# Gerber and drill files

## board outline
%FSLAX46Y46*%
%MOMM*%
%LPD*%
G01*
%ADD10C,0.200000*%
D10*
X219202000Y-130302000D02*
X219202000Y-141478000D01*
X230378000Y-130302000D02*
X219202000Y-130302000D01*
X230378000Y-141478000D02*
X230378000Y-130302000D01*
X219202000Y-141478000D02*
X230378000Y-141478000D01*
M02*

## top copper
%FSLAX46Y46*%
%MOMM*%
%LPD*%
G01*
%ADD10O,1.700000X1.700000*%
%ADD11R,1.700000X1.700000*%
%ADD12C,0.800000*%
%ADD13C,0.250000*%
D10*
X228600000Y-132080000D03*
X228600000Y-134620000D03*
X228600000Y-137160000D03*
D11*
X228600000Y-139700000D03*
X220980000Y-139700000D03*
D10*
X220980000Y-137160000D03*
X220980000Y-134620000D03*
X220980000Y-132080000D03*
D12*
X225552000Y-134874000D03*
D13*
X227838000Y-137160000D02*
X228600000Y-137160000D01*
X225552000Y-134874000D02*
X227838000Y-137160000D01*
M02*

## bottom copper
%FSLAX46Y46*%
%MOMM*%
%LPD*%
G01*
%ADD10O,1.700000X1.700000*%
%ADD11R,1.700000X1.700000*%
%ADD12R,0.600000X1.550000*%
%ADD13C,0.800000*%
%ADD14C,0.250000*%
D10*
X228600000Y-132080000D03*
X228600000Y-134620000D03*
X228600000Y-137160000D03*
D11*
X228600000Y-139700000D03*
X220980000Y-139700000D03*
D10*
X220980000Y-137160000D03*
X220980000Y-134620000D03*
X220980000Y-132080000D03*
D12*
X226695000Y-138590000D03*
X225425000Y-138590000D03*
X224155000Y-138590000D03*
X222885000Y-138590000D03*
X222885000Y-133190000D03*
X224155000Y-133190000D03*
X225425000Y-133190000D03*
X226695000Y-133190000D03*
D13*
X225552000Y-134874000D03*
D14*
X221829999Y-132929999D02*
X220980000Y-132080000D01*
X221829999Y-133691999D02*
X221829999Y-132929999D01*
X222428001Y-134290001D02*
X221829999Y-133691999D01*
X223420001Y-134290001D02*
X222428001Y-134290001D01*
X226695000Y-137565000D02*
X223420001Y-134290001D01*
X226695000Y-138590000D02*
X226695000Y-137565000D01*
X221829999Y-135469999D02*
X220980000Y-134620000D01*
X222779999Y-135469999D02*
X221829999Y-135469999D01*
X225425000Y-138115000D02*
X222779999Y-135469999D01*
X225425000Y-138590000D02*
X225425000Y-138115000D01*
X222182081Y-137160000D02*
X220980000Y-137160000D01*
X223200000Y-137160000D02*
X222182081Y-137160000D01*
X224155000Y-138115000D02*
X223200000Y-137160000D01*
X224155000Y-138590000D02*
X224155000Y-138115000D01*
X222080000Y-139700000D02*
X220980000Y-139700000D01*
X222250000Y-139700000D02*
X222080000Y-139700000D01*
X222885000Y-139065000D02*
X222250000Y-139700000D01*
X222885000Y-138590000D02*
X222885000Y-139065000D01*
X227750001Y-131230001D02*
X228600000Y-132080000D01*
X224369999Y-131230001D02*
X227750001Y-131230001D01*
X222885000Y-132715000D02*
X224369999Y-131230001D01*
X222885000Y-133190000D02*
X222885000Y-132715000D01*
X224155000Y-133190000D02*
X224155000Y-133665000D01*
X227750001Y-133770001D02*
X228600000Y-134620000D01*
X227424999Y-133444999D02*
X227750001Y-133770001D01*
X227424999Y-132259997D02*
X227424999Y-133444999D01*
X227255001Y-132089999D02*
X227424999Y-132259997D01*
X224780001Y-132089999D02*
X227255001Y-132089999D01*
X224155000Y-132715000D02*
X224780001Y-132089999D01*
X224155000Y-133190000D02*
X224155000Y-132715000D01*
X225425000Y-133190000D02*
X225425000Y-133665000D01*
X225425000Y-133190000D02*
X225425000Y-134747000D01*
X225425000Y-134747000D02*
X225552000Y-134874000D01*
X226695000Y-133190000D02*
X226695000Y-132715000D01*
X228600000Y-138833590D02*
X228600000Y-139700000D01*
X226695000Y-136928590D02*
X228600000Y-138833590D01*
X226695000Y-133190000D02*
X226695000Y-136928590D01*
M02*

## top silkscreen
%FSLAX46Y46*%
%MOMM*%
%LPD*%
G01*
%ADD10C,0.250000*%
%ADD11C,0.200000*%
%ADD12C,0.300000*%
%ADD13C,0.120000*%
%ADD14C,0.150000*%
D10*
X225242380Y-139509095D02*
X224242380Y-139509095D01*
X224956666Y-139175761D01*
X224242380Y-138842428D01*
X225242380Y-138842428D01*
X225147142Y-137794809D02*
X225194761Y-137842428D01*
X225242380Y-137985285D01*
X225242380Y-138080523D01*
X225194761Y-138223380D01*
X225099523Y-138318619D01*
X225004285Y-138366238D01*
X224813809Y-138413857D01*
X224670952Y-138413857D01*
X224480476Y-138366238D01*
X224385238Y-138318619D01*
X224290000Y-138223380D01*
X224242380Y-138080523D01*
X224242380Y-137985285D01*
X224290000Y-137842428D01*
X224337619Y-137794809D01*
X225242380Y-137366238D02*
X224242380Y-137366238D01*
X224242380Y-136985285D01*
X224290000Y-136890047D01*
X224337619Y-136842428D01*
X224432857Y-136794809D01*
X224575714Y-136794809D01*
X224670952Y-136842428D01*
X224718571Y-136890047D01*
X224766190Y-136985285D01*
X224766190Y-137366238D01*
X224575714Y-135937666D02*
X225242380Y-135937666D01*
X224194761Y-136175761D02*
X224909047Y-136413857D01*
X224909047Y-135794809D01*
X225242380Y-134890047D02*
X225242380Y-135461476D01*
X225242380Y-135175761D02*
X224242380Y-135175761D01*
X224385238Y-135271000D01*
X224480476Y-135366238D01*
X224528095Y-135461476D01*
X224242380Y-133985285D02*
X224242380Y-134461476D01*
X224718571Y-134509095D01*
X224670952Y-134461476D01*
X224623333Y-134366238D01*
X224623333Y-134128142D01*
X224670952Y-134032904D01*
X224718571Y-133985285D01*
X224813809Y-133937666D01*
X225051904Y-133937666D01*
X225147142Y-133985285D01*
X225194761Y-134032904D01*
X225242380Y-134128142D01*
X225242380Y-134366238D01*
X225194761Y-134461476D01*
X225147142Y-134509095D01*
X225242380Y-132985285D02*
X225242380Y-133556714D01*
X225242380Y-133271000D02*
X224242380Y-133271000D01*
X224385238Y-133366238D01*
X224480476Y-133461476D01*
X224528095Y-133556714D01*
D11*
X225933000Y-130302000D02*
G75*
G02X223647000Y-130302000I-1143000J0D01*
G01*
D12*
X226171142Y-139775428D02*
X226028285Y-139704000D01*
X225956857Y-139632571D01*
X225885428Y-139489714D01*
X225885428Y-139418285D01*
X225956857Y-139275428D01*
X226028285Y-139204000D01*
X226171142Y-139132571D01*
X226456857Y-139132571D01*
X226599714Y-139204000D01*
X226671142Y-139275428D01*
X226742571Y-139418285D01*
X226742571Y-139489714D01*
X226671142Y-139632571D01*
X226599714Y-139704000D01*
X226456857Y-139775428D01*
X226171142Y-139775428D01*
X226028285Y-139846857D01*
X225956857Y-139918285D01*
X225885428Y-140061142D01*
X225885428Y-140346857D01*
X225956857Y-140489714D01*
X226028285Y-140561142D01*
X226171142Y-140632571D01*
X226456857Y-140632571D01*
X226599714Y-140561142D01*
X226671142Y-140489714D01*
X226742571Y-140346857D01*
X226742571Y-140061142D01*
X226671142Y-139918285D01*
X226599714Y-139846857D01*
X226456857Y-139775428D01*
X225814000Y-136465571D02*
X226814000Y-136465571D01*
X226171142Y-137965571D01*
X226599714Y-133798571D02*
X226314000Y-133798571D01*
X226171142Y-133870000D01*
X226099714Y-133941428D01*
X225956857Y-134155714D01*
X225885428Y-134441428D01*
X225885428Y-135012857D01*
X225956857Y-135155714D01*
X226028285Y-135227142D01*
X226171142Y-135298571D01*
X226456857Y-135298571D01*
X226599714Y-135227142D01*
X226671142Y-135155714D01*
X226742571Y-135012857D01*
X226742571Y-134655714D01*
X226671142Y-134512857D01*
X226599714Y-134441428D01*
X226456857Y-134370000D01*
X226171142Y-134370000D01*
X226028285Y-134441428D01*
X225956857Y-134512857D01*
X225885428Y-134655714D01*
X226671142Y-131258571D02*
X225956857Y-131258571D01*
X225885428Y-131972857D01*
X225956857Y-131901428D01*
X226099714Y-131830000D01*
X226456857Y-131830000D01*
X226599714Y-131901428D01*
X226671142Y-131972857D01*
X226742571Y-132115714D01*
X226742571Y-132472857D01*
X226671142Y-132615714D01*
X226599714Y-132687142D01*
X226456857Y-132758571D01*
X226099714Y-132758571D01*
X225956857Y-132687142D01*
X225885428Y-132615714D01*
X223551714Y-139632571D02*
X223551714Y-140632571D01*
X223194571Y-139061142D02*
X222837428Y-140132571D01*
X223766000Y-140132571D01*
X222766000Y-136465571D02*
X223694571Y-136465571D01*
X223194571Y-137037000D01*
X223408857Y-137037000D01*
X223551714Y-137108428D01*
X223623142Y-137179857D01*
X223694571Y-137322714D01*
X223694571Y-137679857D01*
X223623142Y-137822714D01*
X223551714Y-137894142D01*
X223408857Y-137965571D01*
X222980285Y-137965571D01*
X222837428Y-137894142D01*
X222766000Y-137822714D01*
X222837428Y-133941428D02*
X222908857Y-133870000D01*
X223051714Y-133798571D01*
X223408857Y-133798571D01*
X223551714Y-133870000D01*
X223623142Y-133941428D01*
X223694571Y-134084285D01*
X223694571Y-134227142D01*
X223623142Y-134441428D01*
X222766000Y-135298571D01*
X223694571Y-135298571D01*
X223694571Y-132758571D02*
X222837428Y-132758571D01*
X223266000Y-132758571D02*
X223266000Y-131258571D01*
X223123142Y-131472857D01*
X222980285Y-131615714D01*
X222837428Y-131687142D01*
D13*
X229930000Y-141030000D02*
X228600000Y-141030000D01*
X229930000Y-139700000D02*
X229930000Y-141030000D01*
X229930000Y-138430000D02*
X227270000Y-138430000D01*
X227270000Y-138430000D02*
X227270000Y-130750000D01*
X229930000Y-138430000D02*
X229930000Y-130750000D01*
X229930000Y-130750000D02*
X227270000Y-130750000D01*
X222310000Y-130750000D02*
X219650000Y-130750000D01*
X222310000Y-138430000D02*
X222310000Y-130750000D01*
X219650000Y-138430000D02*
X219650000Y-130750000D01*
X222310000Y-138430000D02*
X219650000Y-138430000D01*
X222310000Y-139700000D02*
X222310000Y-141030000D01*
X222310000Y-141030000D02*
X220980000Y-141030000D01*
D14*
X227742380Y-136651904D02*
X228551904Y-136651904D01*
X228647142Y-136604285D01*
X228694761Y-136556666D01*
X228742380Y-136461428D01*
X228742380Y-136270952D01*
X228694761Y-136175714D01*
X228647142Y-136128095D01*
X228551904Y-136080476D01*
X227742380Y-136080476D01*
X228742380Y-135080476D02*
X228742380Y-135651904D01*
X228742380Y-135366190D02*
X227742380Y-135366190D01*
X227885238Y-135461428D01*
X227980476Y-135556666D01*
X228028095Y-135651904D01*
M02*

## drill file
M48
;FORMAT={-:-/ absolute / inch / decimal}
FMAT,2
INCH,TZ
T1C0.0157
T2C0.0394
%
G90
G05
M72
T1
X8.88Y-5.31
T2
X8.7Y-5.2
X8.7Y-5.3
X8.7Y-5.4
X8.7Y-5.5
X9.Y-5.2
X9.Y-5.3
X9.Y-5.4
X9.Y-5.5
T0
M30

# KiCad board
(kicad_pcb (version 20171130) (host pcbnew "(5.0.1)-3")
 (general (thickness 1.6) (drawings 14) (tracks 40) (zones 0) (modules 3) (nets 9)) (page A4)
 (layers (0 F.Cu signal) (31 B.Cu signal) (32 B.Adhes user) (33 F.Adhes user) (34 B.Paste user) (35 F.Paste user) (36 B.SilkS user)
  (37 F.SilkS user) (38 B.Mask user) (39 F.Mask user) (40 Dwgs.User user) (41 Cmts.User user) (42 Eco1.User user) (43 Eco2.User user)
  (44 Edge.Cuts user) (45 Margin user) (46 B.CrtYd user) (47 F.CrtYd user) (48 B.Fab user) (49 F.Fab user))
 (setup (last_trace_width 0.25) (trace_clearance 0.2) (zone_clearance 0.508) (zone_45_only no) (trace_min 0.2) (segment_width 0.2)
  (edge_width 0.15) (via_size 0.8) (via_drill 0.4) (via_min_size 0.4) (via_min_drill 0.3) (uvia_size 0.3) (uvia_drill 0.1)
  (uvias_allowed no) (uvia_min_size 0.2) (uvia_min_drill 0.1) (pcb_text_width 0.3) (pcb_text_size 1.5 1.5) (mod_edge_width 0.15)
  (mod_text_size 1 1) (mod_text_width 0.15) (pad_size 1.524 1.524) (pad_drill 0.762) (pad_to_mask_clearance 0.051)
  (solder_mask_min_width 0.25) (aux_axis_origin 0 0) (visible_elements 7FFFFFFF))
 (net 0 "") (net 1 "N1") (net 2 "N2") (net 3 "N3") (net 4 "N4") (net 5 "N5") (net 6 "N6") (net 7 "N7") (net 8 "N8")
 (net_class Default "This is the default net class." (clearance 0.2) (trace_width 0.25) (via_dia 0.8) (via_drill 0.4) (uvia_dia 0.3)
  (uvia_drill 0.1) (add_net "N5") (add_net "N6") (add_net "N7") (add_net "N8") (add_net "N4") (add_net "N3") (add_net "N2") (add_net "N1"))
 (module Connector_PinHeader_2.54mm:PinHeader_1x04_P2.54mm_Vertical (layer F.Cu) (at 228.6 139.7 180)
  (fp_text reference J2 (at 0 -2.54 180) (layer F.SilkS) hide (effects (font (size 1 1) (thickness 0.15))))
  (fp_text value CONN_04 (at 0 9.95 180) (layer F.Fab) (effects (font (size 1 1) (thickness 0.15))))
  (fp_line (start -1.33 -1.33) (end 0 -1.33) (layer F.SilkS) (width 0.12))
  (fp_line (start -1.33 0) (end -1.33 -1.33) (layer F.SilkS) (width 0.12))
  (fp_line (start -1.33 1.27) (end 1.33 1.27) (layer F.SilkS) (width 0.12))
  (fp_line (start 1.33 1.27) (end 1.33 8.95) (layer F.SilkS) (width 0.12))
  (fp_line (start -1.33 1.27) (end -1.33 8.95) (layer F.SilkS) (width 0.12))
  (fp_line (start -1.33 8.95) (end 1.33 8.95) (layer F.SilkS) (width 0.12))
  (pad 4 thru_hole oval (at 0 7.62 180) (size 1.7 1.7) (drill 1) (layers *.Cu *.Mask) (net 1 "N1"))
  (pad 3 thru_hole oval (at 0 5.08 180) (size 1.7 1.7) (drill 1) (layers *.Cu *.Mask) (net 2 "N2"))
  (pad 2 thru_hole oval (at 0 2.54 180) (size 1.7 1.7) (drill 1) (layers *.Cu *.Mask) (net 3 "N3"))
  (pad 1 thru_hole rect (at 0 0 180) (size 1.7 1.7) (drill 1) (layers *.Cu *.Mask) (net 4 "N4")))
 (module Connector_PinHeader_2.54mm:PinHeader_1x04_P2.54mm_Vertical (layer F.Cu) (at 220.98 139.7 180)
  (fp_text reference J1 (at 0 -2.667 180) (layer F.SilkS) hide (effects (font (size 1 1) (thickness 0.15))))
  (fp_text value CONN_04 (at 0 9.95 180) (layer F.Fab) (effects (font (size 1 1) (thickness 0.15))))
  (fp_line (start -1.33 8.95) (end 1.33 8.95) (layer F.SilkS) (width 0.12))
  (fp_line (start -1.33 1.27) (end -1.33 8.95) (layer F.SilkS) (width 0.12))
  (fp_line (start 1.33 1.27) (end 1.33 8.95) (layer F.SilkS) (width 0.12))
  (fp_line (start -1.33 1.27) (end 1.33 1.27) (layer F.SilkS) (width 0.12))
  (fp_line (start -1.33 0) (end -1.33 -1.33) (layer F.SilkS) (width 0.12))
  (fp_line (start -1.33 -1.33) (end 0 -1.33) (layer F.SilkS) (width 0.12))
  (pad 1 thru_hole rect (at 0 0 180) (size 1.7 1.7) (drill 1) (layers *.Cu *.Mask) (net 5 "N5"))
  (pad 2 thru_hole oval (at 0 2.54 180) (size 1.7 1.7) (drill 1) (layers *.Cu *.Mask) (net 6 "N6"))
  (pad 3 thru_hole oval (at 0 5.08 180) (size 1.7 1.7) (drill 1) (layers *.Cu *.Mask) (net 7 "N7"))
  (pad 4 thru_hole oval (at 0 7.62 180) (size 1.7 1.7) (drill 1) (layers *.Cu *.Mask) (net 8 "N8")))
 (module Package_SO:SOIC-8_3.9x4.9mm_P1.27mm (layer B.Cu) (at 224.79 135.89 90)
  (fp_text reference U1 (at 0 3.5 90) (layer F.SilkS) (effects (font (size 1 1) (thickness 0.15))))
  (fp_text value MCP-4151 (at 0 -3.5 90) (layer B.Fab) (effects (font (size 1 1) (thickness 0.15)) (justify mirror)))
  (pad 1 smd rect (at -2.7 1.905 90) (size 1.55 0.6) (layers B.Cu B.Paste B.Mask) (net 8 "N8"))
  (pad 2 smd rect (at -2.7 0.635 90) (size 1.55 0.6) (layers B.Cu B.Paste B.Mask) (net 7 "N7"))
  (pad 3 smd rect (at -2.7 -0.635 90) (size 1.55 0.6) (layers B.Cu B.Paste B.Mask) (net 6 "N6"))
  (pad 4 smd rect (at -2.7 -1.905 90) (size 1.55 0.6) (layers B.Cu B.Paste B.Mask) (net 5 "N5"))
  (pad 5 smd rect (at 2.7 -1.905 90) (size 1.55 0.6) (layers B.Cu B.Paste B.Mask) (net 1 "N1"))
  (pad 6 smd rect (at 2.7 -0.635 90) (size 1.55 0.6) (layers B.Cu B.Paste B.Mask) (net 2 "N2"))
  (pad 7 smd rect (at 2.7 0.635 90) (size 1.55 0.6) (layers B.Cu B.Paste B.Mask) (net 3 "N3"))
  (pad 8 smd rect (at 2.7 1.905 90) (size 1.55 0.6) (layers B.Cu B.Paste B.Mask) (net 4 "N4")))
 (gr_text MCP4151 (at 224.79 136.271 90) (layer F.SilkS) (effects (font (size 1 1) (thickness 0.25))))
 (gr_arc (start 224.79 130.302) (end 223.647 130.302) (angle -180) (layer F.SilkS) (width 0.2))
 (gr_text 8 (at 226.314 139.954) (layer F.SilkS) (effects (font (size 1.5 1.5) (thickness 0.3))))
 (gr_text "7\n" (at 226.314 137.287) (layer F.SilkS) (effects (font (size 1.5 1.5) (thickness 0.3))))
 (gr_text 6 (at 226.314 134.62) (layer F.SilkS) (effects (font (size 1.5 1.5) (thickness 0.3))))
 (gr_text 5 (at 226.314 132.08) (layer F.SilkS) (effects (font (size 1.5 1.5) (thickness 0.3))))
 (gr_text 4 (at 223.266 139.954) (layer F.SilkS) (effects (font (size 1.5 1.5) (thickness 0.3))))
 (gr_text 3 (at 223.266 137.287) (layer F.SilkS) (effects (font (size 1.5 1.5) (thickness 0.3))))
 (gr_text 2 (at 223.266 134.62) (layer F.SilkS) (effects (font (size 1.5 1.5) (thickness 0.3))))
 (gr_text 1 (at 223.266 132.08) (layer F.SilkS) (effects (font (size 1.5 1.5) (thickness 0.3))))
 (gr_line (start 219.202 130.302) (end 219.202 141.478) (layer Edge.Cuts) (width 0.2))
 (gr_line (start 230.378 130.302) (end 219.202 130.302) (layer Edge.Cuts) (width 0.2))
 (gr_line (start 230.378 141.478) (end 230.378 130.302) (layer Edge.Cuts) (width 0.2))
 (gr_line (start 219.202 141.478) (end 230.378 141.478) (layer Edge.Cuts) (width 0.2))
 (segment (start 221.829999 132.929999) (end 220.98 132.08) (width 0.25) (layer B.Cu) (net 8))
 (segment (start 221.829999 133.691999) (end 221.829999 132.929999) (width 0.25) (layer B.Cu) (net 8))
 (segment (start 222.428001 134.290001) (end 221.829999 133.691999) (width 0.25) (layer B.Cu) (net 8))
 (segment (start 223.420001 134.290001) (end 222.428001 134.290001) (width 0.25) (layer B.Cu) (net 8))
 (segment (start 226.695 137.565) (end 223.420001 134.290001) (width 0.25) (layer B.Cu) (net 8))
 (segment (start 226.695 138.59) (end 226.695 137.565) (width 0.25) (layer B.Cu) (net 8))
 (segment (start 221.829999 135.469999) (end 220.98 134.62) (width 0.25) (layer B.Cu) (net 7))
 (segment (start 222.779999 135.469999) (end 221.829999 135.469999) (width 0.25) (layer B.Cu) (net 7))
 (segment (start 225.425 138.115) (end 222.779999 135.469999) (width 0.25) (layer B.Cu) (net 7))
 (segment (start 225.425 138.59) (end 225.425 138.115) (width 0.25) (layer B.Cu) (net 7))
 (segment (start 222.182081 137.16) (end 220.98 137.16) (width 0.25) (layer B.Cu) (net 6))
 (segment (start 223.2 137.16) (end 222.182081 137.16) (width 0.25) (layer B.Cu) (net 6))
 (segment (start 224.155 138.115) (end 223.2 137.16) (width 0.25) (layer B.Cu) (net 6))
 (segment (start 224.155 138.59) (end 224.155 138.115) (width 0.25) (layer B.Cu) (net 6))
 (segment (start 222.08 139.7) (end 220.98 139.7) (width 0.25) (layer B.Cu) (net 5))
 (segment (start 222.25 139.7) (end 222.08 139.7) (width 0.25) (layer B.Cu) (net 5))
 (segment (start 222.885 139.065) (end 222.25 139.7) (width 0.25) (layer B.Cu) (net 5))
 (segment (start 222.885 138.59) (end 222.885 139.065) (width 0.25) (layer B.Cu) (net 5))
 (segment (start 227.750001 131.230001) (end 228.6 132.08) (width 0.25) (layer B.Cu) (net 1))
 (segment (start 224.369999 131.230001) (end 227.750001 131.230001) (width 0.25) (layer B.Cu) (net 1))
 (segment (start 222.885 132.715) (end 224.369999 131.230001) (width 0.25) (layer B.Cu) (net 1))
 (segment (start 222.885 133.19) (end 222.885 132.715) (width 0.25) (layer B.Cu) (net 1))
 (segment (start 224.155 133.19) (end 224.155 133.665) (width 0.25) (layer B.Cu) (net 2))
 (segment (start 227.750001 133.770001) (end 228.6 134.62) (width 0.25) (layer B.Cu) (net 2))
 (segment (start 227.424999 133.444999) (end 227.750001 133.770001) (width 0.25) (layer B.Cu) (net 2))
 (segment (start 227.424999 132.259997) (end 227.424999 133.444999) (width 0.25) (layer B.Cu) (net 2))
 (segment (start 227.255001 132.089999) (end 227.424999 132.259997) (width 0.25) (layer B.Cu) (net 2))
 (segment (start 224.780001 132.089999) (end 227.255001 132.089999) (width 0.25) (layer B.Cu) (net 2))
 (segment (start 224.155 132.715) (end 224.780001 132.089999) (width 0.25) (layer B.Cu) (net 2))
 (segment (start 224.155 133.19) (end 224.155 132.715) (width 0.25) (layer B.Cu) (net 2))
 (segment (start 225.425 133.19) (end 225.425 133.665) (width 0.25) (layer B.Cu) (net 3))
 (via (at 225.552 134.874) (size 0.8) (drill 0.4) (layers F.Cu B.Cu) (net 3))
 (segment (start 225.425 133.19) (end 225.425 134.747) (width 0.25) (layer B.Cu) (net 3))
 (segment (start 225.425 134.747) (end 225.552 134.874) (width 0.25) (layer B.Cu) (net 3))
 (segment (start 227.838 137.16) (end 228.6 137.16) (width 0.25) (layer F.Cu) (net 3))
 (segment (start 225.552 134.874) (end 227.838 137.16) (width 0.25) (layer F.Cu) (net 3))
 (segment (start 226.695 133.19) (end 226.695 132.715) (width 0.25) (layer B.Cu) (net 4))
 (segment (start 228.6 138.83359) (end 228.6 139.7) (width 0.25) (layer B.Cu) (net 4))
 (segment (start 226.695 136.92859) (end 228.6 138.83359) (width 0.25) (layer B.Cu) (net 4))
 (segment (start 226.695 133.19) (end 226.695 136.92859) (width 0.25) (layer B.Cu) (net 4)))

